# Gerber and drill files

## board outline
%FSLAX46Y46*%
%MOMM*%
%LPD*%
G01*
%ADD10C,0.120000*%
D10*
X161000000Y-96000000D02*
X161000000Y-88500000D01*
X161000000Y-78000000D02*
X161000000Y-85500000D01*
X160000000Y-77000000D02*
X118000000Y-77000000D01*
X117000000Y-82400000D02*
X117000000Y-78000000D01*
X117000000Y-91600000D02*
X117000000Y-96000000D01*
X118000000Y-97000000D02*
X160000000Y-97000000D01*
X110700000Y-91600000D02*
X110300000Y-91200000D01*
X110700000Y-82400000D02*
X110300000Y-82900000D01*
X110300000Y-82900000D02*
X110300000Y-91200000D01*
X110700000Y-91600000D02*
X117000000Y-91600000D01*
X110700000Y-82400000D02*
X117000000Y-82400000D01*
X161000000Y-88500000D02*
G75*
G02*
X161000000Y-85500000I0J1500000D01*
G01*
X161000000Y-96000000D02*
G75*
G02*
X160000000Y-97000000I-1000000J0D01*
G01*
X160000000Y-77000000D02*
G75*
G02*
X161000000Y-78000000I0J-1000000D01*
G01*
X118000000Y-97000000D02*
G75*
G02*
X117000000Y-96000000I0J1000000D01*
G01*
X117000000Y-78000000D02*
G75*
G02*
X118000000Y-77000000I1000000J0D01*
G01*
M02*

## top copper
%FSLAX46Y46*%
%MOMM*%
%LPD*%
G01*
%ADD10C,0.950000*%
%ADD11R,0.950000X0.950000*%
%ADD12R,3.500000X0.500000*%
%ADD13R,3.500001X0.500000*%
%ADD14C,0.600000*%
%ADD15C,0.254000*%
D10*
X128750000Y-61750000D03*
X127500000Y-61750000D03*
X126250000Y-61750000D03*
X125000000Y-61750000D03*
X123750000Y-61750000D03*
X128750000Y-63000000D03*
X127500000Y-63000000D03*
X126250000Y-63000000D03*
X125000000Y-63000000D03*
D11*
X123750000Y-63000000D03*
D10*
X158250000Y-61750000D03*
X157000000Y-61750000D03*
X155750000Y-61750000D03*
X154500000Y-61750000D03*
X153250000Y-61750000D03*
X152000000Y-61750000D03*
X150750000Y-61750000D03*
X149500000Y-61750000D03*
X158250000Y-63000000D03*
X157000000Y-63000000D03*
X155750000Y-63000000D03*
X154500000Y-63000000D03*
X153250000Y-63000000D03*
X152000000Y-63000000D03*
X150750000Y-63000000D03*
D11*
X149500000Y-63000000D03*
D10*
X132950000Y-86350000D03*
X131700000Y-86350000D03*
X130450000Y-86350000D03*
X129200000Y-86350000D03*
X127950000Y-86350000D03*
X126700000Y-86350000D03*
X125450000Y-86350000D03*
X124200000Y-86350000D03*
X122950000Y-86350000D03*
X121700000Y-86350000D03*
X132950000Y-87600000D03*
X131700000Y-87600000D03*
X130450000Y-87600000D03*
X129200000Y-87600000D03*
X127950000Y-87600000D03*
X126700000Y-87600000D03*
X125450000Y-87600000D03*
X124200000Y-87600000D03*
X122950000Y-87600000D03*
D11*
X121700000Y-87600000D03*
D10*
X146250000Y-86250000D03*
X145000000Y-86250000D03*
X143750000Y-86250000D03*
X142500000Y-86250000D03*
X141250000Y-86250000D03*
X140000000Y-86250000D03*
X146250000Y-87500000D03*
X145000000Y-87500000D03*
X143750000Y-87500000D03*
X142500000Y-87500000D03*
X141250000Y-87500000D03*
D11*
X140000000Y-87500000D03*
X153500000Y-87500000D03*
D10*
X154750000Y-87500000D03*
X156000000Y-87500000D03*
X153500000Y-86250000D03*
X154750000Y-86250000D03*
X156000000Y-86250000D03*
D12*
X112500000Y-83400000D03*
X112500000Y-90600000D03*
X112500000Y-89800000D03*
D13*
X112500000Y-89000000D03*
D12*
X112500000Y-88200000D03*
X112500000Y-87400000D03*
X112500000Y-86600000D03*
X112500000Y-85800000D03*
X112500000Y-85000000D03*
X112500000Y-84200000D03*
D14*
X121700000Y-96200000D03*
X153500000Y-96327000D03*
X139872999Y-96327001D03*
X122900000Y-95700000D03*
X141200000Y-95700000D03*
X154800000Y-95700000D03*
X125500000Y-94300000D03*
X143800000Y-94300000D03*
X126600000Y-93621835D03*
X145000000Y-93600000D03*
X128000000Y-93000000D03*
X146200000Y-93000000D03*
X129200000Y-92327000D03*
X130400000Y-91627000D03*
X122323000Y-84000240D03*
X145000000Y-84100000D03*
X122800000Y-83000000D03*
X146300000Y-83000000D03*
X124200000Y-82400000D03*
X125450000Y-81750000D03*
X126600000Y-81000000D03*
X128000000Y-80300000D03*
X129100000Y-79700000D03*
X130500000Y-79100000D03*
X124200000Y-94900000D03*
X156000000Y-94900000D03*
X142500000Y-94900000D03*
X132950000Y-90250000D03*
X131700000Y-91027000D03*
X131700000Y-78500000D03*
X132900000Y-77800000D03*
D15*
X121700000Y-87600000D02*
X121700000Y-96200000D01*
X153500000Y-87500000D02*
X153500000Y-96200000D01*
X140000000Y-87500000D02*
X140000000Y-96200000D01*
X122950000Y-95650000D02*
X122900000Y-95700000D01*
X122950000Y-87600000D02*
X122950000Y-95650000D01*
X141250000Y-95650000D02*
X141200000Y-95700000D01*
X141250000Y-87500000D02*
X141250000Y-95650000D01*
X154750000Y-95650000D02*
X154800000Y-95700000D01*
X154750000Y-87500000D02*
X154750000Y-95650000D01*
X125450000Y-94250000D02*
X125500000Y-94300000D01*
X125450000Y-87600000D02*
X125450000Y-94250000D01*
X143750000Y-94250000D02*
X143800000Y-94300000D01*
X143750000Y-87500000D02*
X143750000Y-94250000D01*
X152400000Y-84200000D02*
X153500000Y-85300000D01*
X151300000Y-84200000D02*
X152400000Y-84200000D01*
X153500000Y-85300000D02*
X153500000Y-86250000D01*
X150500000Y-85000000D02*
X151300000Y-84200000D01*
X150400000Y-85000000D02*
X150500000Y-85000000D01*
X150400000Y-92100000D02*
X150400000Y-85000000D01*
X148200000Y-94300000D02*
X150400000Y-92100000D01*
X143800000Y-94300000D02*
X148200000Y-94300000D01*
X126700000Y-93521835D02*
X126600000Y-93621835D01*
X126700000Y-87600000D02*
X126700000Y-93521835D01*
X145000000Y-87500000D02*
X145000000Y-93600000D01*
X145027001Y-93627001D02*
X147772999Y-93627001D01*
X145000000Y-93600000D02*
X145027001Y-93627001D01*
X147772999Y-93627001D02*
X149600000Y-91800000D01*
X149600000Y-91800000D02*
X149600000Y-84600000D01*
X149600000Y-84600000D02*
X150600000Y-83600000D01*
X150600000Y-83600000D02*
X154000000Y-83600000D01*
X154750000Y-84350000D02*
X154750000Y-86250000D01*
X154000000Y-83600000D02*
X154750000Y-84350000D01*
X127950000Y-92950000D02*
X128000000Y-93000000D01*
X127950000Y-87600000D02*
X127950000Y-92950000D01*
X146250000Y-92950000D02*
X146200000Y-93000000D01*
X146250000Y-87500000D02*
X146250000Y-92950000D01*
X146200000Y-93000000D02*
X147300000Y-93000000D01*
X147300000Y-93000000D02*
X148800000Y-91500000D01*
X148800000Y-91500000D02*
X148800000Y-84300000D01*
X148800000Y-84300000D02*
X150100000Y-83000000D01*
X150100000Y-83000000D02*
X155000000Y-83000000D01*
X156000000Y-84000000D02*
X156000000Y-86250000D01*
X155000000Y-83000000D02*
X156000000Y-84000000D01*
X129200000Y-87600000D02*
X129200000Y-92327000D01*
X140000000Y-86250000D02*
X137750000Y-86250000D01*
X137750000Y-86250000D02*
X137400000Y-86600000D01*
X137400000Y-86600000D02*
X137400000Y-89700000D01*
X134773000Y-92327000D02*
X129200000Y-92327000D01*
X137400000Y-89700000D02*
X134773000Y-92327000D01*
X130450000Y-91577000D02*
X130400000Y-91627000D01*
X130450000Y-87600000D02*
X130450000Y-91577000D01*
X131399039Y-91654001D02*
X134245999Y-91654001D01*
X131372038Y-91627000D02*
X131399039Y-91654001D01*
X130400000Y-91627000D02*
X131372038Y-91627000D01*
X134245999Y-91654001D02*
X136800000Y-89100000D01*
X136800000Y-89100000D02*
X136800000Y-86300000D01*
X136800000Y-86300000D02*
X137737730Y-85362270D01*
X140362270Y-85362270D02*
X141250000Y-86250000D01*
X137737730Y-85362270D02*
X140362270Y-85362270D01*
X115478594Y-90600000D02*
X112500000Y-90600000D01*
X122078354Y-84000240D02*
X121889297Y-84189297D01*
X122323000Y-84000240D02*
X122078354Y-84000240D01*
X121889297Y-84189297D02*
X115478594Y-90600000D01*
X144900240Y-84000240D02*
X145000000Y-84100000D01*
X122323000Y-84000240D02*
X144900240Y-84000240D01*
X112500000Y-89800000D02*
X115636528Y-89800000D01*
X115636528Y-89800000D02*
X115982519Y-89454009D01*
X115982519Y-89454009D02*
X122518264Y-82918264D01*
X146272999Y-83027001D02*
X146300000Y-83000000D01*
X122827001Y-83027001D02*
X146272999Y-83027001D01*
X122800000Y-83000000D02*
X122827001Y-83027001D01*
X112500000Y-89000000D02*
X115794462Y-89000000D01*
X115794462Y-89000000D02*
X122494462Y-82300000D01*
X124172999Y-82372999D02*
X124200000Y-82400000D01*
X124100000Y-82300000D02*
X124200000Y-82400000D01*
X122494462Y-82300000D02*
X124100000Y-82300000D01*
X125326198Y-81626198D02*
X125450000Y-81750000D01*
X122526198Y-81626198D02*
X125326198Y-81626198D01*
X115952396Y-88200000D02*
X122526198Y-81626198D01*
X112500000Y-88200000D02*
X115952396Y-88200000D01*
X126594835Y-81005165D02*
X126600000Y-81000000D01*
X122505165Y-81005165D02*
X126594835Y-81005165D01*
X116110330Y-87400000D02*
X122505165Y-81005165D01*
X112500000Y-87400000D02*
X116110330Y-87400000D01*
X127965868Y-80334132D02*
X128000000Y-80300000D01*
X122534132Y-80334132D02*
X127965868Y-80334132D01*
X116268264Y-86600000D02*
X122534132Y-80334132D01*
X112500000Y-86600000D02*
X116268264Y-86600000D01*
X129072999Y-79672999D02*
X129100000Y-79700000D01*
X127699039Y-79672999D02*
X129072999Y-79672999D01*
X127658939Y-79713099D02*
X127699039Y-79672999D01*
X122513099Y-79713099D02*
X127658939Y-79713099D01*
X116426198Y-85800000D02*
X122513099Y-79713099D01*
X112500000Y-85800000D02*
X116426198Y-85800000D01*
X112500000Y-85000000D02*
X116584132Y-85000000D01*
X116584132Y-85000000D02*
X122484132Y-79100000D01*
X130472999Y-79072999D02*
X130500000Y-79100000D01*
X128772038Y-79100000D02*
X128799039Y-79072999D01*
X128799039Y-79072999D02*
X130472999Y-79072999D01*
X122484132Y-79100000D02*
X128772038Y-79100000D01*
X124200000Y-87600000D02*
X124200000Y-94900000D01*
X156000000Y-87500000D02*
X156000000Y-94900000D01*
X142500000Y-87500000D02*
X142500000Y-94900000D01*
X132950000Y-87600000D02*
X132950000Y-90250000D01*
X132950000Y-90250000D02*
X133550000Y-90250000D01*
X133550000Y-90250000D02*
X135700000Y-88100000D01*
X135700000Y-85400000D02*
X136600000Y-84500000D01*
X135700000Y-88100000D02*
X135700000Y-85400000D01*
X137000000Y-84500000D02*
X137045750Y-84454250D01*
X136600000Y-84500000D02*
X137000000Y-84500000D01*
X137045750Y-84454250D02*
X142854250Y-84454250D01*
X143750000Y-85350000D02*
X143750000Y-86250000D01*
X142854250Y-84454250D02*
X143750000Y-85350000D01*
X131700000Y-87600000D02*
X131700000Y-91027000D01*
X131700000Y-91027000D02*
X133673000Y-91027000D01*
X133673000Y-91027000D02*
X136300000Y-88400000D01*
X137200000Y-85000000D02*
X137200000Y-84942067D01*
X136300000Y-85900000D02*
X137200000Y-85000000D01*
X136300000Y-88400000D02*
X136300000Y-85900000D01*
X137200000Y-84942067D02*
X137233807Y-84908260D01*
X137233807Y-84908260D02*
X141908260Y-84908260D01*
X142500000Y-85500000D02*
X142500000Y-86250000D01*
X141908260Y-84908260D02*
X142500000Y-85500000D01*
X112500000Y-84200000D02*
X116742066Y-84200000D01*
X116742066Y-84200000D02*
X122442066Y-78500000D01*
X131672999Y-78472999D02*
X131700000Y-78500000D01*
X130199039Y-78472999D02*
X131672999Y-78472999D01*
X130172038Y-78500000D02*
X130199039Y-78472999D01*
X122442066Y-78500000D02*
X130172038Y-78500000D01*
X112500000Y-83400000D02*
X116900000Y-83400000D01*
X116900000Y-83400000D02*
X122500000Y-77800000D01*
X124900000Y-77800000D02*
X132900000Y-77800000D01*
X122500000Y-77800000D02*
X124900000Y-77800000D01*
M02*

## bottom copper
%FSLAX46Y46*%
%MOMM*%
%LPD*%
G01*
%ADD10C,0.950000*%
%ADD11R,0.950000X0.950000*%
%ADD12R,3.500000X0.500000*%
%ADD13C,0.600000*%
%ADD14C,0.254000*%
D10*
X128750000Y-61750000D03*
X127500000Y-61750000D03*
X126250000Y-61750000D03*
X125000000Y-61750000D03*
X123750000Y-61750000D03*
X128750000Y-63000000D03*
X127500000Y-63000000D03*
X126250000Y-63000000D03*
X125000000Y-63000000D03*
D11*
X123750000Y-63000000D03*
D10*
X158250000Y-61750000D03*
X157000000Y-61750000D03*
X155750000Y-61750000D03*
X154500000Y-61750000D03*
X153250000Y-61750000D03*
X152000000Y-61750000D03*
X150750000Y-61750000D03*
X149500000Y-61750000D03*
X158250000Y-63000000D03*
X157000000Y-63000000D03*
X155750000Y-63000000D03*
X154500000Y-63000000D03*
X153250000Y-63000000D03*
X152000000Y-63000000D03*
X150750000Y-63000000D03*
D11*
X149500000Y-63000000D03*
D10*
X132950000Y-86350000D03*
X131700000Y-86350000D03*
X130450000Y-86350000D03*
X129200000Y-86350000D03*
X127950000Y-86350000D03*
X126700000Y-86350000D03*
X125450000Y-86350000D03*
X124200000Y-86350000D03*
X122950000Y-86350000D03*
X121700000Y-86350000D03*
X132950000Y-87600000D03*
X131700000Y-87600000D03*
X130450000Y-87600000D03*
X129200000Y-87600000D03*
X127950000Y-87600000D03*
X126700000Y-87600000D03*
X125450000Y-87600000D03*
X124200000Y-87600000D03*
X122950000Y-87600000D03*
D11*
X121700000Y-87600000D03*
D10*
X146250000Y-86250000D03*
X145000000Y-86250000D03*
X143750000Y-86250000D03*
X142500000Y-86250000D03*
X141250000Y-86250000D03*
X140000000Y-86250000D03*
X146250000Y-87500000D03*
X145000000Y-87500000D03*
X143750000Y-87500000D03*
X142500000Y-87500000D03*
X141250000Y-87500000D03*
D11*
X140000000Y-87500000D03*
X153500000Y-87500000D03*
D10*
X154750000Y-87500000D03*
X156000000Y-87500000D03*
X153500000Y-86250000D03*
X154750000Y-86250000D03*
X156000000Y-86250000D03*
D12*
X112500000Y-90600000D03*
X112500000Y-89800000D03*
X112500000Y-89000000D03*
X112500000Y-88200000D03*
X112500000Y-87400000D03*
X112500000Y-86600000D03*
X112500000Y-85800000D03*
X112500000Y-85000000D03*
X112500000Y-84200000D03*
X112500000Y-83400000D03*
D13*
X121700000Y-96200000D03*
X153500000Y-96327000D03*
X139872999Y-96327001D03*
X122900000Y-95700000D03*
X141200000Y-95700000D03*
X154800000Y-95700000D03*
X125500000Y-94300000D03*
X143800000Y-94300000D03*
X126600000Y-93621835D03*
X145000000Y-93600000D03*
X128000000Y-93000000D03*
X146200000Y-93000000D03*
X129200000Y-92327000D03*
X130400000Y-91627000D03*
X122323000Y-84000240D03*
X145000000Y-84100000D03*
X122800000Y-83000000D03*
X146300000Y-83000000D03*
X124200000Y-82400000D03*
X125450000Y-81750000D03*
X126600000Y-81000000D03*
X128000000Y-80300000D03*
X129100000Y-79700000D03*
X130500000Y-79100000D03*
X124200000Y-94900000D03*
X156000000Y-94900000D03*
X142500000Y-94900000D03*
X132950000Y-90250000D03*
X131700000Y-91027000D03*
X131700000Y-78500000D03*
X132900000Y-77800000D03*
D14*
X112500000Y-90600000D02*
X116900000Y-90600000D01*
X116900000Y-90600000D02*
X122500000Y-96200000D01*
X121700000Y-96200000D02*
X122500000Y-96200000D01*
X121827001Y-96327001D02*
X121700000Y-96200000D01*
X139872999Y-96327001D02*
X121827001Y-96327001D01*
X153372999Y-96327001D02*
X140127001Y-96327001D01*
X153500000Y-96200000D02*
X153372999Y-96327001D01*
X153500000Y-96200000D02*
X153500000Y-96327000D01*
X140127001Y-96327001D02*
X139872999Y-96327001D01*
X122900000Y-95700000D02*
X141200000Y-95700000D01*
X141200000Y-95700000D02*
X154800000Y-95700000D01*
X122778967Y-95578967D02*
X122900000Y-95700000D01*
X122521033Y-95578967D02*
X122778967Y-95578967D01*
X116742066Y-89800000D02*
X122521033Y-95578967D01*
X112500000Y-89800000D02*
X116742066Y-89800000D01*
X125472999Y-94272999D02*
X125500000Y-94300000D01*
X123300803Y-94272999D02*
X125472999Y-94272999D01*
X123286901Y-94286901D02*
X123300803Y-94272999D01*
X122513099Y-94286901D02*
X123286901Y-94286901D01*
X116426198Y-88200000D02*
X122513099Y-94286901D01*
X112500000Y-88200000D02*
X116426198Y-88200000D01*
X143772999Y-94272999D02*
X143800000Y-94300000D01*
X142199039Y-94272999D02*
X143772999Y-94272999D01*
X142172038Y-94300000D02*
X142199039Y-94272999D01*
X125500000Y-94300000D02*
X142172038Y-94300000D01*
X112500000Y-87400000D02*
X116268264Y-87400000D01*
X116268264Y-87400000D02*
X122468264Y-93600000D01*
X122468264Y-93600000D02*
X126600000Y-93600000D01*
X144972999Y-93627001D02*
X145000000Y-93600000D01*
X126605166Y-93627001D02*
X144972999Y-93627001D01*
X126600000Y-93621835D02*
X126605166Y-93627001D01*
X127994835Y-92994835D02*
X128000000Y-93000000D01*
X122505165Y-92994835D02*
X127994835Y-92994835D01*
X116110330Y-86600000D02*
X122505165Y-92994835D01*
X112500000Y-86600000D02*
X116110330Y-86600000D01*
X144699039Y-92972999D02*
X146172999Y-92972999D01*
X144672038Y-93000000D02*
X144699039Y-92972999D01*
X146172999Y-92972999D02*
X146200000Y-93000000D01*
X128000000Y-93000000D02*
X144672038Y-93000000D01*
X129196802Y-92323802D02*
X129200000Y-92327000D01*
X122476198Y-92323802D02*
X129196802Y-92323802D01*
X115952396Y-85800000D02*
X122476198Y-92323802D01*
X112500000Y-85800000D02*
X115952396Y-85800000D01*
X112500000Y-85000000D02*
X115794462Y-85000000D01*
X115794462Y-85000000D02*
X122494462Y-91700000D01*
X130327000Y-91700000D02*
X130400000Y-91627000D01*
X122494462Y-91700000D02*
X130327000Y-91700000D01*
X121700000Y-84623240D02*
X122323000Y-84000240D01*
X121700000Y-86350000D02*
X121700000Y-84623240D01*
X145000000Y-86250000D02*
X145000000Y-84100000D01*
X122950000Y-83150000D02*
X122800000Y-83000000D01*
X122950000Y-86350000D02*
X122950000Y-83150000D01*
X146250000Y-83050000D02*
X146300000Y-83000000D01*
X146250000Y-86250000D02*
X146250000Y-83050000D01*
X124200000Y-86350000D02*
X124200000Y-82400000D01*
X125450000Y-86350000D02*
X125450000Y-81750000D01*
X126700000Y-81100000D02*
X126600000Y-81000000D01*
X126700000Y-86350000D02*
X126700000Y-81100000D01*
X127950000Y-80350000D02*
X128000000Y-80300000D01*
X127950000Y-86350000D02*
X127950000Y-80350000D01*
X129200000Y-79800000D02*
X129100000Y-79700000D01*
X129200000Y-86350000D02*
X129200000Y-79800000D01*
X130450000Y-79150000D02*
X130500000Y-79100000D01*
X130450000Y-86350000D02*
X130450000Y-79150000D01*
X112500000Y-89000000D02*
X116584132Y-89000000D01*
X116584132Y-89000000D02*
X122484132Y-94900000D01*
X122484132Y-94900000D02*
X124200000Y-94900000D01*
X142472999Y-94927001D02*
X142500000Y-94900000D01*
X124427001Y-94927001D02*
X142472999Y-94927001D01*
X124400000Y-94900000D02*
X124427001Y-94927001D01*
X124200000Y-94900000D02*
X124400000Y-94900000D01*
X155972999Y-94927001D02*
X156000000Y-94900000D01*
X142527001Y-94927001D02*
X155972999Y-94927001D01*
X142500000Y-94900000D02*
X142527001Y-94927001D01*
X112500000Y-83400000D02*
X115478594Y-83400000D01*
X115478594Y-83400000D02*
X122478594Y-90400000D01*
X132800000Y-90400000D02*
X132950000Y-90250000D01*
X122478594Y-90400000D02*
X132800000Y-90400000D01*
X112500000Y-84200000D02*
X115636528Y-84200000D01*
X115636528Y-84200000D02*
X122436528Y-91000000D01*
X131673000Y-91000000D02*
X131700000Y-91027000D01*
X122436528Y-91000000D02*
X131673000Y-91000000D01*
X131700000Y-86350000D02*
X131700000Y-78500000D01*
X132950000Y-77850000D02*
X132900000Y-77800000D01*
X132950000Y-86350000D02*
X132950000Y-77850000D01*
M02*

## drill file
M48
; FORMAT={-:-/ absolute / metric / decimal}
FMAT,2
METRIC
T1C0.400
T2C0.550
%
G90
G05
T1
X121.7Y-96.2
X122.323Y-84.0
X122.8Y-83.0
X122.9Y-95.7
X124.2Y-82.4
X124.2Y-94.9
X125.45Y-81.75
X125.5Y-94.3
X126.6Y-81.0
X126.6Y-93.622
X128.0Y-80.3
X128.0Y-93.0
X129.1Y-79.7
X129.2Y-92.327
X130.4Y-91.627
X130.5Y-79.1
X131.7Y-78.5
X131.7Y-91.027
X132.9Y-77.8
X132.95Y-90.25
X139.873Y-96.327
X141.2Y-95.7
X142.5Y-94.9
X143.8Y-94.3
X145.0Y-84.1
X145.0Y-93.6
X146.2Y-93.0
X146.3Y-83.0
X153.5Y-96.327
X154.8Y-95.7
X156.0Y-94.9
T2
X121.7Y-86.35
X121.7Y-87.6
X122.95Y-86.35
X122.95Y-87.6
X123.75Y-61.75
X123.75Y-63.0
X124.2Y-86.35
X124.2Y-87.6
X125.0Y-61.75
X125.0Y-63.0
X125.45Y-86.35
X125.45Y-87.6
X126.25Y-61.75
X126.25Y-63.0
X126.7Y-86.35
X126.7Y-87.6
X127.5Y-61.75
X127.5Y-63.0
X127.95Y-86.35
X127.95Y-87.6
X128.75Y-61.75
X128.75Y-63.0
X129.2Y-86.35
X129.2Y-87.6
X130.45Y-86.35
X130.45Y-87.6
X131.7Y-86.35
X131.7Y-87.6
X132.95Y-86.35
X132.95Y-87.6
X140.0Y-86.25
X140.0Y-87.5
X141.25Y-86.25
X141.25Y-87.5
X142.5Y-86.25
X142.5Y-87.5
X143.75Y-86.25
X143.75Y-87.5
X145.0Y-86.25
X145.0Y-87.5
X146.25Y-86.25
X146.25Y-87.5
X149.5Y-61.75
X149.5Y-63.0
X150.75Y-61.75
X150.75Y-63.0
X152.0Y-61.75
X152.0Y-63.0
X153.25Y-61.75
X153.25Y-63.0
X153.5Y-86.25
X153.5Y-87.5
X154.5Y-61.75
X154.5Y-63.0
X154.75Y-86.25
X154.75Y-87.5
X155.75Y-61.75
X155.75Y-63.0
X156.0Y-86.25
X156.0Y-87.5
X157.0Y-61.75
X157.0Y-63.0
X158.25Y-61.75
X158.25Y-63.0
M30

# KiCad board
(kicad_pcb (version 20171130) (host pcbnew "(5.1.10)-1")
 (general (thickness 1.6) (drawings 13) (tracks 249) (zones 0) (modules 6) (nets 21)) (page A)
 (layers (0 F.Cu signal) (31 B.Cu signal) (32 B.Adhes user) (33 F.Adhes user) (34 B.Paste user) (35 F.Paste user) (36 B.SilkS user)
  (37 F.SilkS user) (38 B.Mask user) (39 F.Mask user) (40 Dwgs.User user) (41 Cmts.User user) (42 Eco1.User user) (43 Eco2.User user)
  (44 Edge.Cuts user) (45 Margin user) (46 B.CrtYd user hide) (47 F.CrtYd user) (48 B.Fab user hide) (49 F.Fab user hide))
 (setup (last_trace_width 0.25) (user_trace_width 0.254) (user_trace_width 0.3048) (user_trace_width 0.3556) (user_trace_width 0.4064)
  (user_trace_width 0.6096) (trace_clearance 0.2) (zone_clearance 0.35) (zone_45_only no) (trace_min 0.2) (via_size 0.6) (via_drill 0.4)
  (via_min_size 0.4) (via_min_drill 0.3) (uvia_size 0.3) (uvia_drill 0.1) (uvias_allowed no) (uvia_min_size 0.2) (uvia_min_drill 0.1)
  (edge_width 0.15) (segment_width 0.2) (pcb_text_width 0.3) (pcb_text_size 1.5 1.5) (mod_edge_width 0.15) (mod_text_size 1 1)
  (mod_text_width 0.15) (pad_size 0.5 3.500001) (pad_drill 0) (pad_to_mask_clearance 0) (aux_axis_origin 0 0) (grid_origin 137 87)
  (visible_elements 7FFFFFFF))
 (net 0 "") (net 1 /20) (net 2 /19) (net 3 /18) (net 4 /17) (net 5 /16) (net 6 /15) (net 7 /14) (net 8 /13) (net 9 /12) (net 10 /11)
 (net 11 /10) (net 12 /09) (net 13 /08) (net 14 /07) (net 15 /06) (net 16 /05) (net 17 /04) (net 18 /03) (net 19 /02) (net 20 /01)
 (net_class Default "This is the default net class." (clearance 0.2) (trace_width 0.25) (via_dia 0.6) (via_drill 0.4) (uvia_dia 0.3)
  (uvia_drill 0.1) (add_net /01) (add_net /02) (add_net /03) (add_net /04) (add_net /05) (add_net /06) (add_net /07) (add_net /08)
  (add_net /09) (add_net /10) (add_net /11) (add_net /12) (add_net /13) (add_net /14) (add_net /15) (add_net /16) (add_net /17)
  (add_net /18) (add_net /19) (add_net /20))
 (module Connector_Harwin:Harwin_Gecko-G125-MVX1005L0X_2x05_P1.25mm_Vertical (layer F.Cu) (at 123.75 63)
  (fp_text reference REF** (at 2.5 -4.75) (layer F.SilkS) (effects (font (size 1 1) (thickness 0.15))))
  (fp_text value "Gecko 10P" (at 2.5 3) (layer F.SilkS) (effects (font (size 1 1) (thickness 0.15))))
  (pad 10 thru_hole circle (at 5 -1.25) (size 0.95 0.95) (drill 0.55) (layers *.Cu *.Mask))
  (pad 9 thru_hole circle (at 3.75 -1.25) (size 0.95 0.95) (drill 0.55) (layers *.Cu *.Mask))
  (pad 8 thru_hole circle (at 2.5 -1.25) (size 0.95 0.95) (drill 0.55) (layers *.Cu *.Mask))
  (pad 7 thru_hole circle (at 1.25 -1.25) (size 0.95 0.95) (drill 0.55) (layers *.Cu *.Mask))
  (pad 6 thru_hole circle (at 0 -1.25) (size 0.95 0.95) (drill 0.55) (layers *.Cu *.Mask))
  (pad 5 thru_hole circle (at 5 0) (size 0.95 0.95) (drill 0.55) (layers *.Cu *.Mask))
  (pad 4 thru_hole circle (at 3.75 0) (size 0.95 0.95) (drill 0.55) (layers *.Cu *.Mask))
  (pad 3 thru_hole circle (at 2.5 0) (size 0.95 0.95) (drill 0.55) (layers *.Cu *.Mask))
  (pad 2 thru_hole circle (at 1.25 0) (size 0.95 0.95) (drill 0.55) (layers *.Cu *.Mask))
  (pad 1 thru_hole rect (at 0 0) (size 0.95 0.95) (drill 0.55) (layers *.Cu *.Mask)))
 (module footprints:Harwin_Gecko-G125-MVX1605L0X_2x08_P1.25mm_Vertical (layer F.Cu) (at 149.5 63)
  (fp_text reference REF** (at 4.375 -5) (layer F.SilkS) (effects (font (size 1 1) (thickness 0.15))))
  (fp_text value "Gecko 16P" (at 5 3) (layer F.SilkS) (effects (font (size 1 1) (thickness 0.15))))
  (pad 16 thru_hole circle (at 8.75 -1.25) (size 0.95 0.95) (drill 0.55) (layers *.Cu *.Mask))
  (pad 15 thru_hole circle (at 7.5 -1.25) (size 0.95 0.95) (drill 0.55) (layers *.Cu *.Mask))
  (pad 14 thru_hole circle (at 6.25 -1.25) (size 0.95 0.95) (drill 0.55) (layers *.Cu *.Mask))
  (pad 13 thru_hole circle (at 5 -1.25) (size 0.95 0.95) (drill 0.55) (layers *.Cu *.Mask))
  (pad 12 thru_hole circle (at 3.75 -1.25) (size 0.95 0.95) (drill 0.55) (layers *.Cu *.Mask))
  (pad 11 thru_hole circle (at 2.5 -1.25) (size 0.95 0.95) (drill 0.55) (layers *.Cu *.Mask))
  (pad 10 thru_hole circle (at 1.25 -1.25) (size 0.95 0.95) (drill 0.55) (layers *.Cu *.Mask))
  (pad 9 thru_hole circle (at 0 -1.25) (size 0.95 0.95) (drill 0.55) (layers *.Cu *.Mask))
  (pad 8 thru_hole circle (at 8.75 0) (size 0.95 0.95) (drill 0.55) (layers *.Cu *.Mask))
  (pad 7 thru_hole circle (at 7.5 0) (size 0.95 0.95) (drill 0.55) (layers *.Cu *.Mask))
  (pad 6 thru_hole circle (at 6.25 0) (size 0.95 0.95) (drill 0.55) (layers *.Cu *.Mask))
  (pad 5 thru_hole circle (at 5 0) (size 0.95 0.95) (drill 0.55) (layers *.Cu *.Mask))
  (pad 4 thru_hole circle (at 3.75 0) (size 0.95 0.95) (drill 0.55) (layers *.Cu *.Mask))
  (pad 3 thru_hole circle (at 2.5 0) (size 0.95 0.95) (drill 0.55) (layers *.Cu *.Mask))
  (pad 2 thru_hole circle (at 1.25 0) (size 0.95 0.95) (drill 0.55) (layers *.Cu *.Mask))
  (pad 1 thru_hole rect (at 0 0) (size 0.95 0.95) (drill 0.55) (layers *.Cu *.Mask)))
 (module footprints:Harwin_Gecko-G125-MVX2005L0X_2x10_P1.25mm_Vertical (layer F.Cu) (at 121.7 87.6)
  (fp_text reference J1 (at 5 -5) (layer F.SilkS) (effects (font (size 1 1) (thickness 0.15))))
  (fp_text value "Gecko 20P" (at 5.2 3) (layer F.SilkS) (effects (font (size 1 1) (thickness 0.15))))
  (pad 20 thru_hole circle (at 11.25 -1.25) (size 0.95 0.95) (drill 0.55) (layers *.Cu *.Mask) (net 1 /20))
  (pad 19 thru_hole circle (at 10 -1.25) (size 0.95 0.95) (drill 0.55) (layers *.Cu *.Mask) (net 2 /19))
  (pad 18 thru_hole circle (at 8.75 -1.25) (size 0.95 0.95) (drill 0.55) (layers *.Cu *.Mask) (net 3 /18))
  (pad 17 thru_hole circle (at 7.5 -1.25) (size 0.95 0.95) (drill 0.55) (layers *.Cu *.Mask) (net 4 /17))
  (pad 16 thru_hole circle (at 6.25 -1.25) (size 0.95 0.95) (drill 0.55) (layers *.Cu *.Mask) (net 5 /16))
  (pad 15 thru_hole circle (at 5 -1.25) (size 0.95 0.95) (drill 0.55) (layers *.Cu *.Mask) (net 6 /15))
  (pad 14 thru_hole circle (at 3.75 -1.25) (size 0.95 0.95) (drill 0.55) (layers *.Cu *.Mask) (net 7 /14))
  (pad 13 thru_hole circle (at 2.5 -1.25) (size 0.95 0.95) (drill 0.55) (layers *.Cu *.Mask) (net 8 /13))
  (pad 12 thru_hole circle (at 1.25 -1.25) (size 0.95 0.95) (drill 0.55) (layers *.Cu *.Mask) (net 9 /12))
  (pad 11 thru_hole circle (at 0 -1.25) (size 0.95 0.95) (drill 0.55) (layers *.Cu *.Mask) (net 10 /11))
  (pad 10 thru_hole circle (at 11.25 0) (size 0.95 0.95) (drill 0.55) (layers *.Cu *.Mask) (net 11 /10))
  (pad 9 thru_hole circle (at 10 0) (size 0.95 0.95) (drill 0.55) (layers *.Cu *.Mask) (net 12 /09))
  (pad 8 thru_hole circle (at 8.75 0) (size 0.95 0.95) (drill 0.55) (layers *.Cu *.Mask) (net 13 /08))
  (pad 7 thru_hole circle (at 7.5 0) (size 0.95 0.95) (drill 0.55) (layers *.Cu *.Mask) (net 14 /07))
  (pad 6 thru_hole circle (at 6.25 0) (size 0.95 0.95) (drill 0.55) (layers *.Cu *.Mask) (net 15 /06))
  (pad 5 thru_hole circle (at 5 0) (size 0.95 0.95) (drill 0.55) (layers *.Cu *.Mask) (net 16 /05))
  (pad 4 thru_hole circle (at 3.75 0) (size 0.95 0.95) (drill 0.55) (layers *.Cu *.Mask) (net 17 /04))
  (pad 3 thru_hole circle (at 2.5 0) (size 0.95 0.95) (drill 0.55) (layers *.Cu *.Mask) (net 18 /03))
  (pad 2 thru_hole circle (at 1.25 0) (size 0.95 0.95) (drill 0.55) (layers *.Cu *.Mask) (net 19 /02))
  (pad 1 thru_hole rect (at 0 0) (size 0.95 0.95) (drill 0.55) (layers *.Cu *.Mask) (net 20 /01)))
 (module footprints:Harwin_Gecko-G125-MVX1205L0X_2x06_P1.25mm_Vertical (layer F.Cu) (at 140 87.5)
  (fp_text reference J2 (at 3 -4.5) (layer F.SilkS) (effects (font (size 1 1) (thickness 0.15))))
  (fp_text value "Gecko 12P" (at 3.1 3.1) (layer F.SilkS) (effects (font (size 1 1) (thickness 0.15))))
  (pad 12 thru_hole circle (at 6.25 -1.25) (size 0.95 0.95) (drill 0.55) (layers *.Cu *.Mask) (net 9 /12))
  (pad 11 thru_hole circle (at 5 -1.25) (size 0.95 0.95) (drill 0.55) (layers *.Cu *.Mask) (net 10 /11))
  (pad 10 thru_hole circle (at 3.75 -1.25) (size 0.95 0.95) (drill 0.55) (layers *.Cu *.Mask) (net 11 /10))
  (pad 9 thru_hole circle (at 2.5 -1.25) (size 0.95 0.95) (drill 0.55) (layers *.Cu *.Mask) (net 12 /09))
  (pad 8 thru_hole circle (at 1.25 -1.25) (size 0.95 0.95) (drill 0.55) (layers *.Cu *.Mask) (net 13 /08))
  (pad 7 thru_hole circle (at 0 -1.25) (size 0.95 0.95) (drill 0.55) (layers *.Cu *.Mask) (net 14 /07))
  (pad 6 thru_hole circle (at 6.25 0) (size 0.95 0.95) (drill 0.55) (layers *.Cu *.Mask) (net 15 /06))
  (pad 5 thru_hole circle (at 5 0) (size 0.95 0.95) (drill 0.55) (layers *.Cu *.Mask) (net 16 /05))
  (pad 4 thru_hole circle (at 3.75 0) (size 0.95 0.95) (drill 0.55) (layers *.Cu *.Mask) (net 17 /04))
  (pad 3 thru_hole circle (at 2.5 0) (size 0.95 0.95) (drill 0.55) (layers *.Cu *.Mask) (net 18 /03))
  (pad 2 thru_hole circle (at 1.25 0) (size 0.95 0.95) (drill 0.55) (layers *.Cu *.Mask) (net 19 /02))
  (pad 1 thru_hole rect (at 0 0) (size 0.95 0.95) (drill 0.55) (layers *.Cu *.Mask) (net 20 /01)))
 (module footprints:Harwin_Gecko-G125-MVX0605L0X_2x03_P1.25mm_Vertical (layer F.Cu) (at 153.5 87.5)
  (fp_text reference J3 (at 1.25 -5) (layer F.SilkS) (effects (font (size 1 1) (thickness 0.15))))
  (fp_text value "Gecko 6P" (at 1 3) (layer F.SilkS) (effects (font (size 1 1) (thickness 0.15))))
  (pad 1 thru_hole rect (at 0 0) (size 0.95 0.95) (drill 0.55) (layers *.Cu *.Mask) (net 20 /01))
  (pad 2 thru_hole circle (at 1.25 0) (size 0.95 0.95) (drill 0.55) (layers *.Cu *.Mask) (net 19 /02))
  (pad 3 thru_hole circle (at 2.5 0) (size 0.95 0.95) (drill 0.55) (layers *.Cu *.Mask) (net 18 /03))
  (pad 4 thru_hole circle (at 0 -1.25) (size 0.95 0.95) (drill 0.55) (layers *.Cu *.Mask) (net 17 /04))
  (pad 5 thru_hole circle (at 1.25 -1.25) (size 0.95 0.95) (drill 0.55) (layers *.Cu *.Mask) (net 16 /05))
  (pad 6 thru_hole circle (at 2.5 -1.25) (size 0.95 0.95) (drill 0.55) (layers *.Cu *.Mask) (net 15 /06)))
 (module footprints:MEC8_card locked (layer F.Cu) (at 112.5 87 90)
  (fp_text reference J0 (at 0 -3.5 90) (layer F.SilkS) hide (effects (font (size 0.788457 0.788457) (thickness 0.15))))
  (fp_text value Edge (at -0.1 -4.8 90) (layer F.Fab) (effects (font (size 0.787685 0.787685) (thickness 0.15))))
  (fp_line (start -9 48.5) (end -1.5 48.5) (layer Edge.Cuts) (width 0.12))
  (fp_line (start 9 48.5) (end 1.5 48.5) (layer Edge.Cuts) (width 0.12))
  (fp_line (start 10 47.5) (end 10 5.5) (layer Edge.Cuts) (width 0.12))
  (fp_line (start 4.6 4.5) (end 9 4.5) (layer Edge.Cuts) (width 0.12))
  (fp_line (start -4.6 4.5) (end -9 4.5) (layer Edge.Cuts) (width 0.12))
  (fp_line (start -10 5.5) (end -10 47.5) (layer Edge.Cuts) (width 0.12))
  (fp_line (start -4.6 -1.8) (end -4.2 -2.2) (layer Edge.Cuts) (width 0.12))
  (fp_line (start 4.6 -1.8) (end 4.1 -2.2) (layer Edge.Cuts) (width 0.12))
  (fp_line (start 4.1 -2.2) (end -4.2 -2.2) (layer Edge.Cuts) (width 0.12))
  (fp_line (start -4.6 -1.8) (end -4.6 4.5) (layer Edge.Cuts) (width 0.12))
  (fp_line (start 4.6 -1.8) (end 4.6 4.5) (layer Edge.Cuts) (width 0.12))
  (fp_arc (start 0 48.5) (end 1.5 48.5) (angle -180) (layer Edge.Cuts) (width 0.12))
  (fp_arc (start -9 47.5) (end -10 47.5) (angle -90) (layer Edge.Cuts) (width 0.12))
  (fp_arc (start 9 47.5) (end 9 48.5) (angle -90) (layer Edge.Cuts) (width 0.12))
  (fp_arc (start -9 5.5) (end -9 4.5) (angle -90) (layer Edge.Cuts) (width 0.12))
  (fp_arc (start 9 5.5) (end 10 5.5) (angle -90) (layer Edge.Cuts) (width 0.12))
  (pad 20 smd rect (at 3.6 0 90) (size 0.5 3.5) (layers F.Cu F.Paste F.Mask) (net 1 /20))
  (pad 11 smd rect (at -3.6 0 90) (size 0.5 3.5) (layers F.Cu F.Paste F.Mask) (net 10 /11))
  (pad 12 smd rect (at -2.8 0 90) (size 0.5 3.5) (layers F.Cu F.Paste F.Mask) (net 9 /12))
  (pad 13 smd rect (at -2 0 90) (size 0.5 3.500001) (layers F.Cu F.Paste F.Mask) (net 8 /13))
  (pad 14 smd rect (at -1.2 0 90) (size 0.5 3.5) (layers F.Cu F.Paste F.Mask) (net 7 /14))
  (pad 15 smd rect (at -0.4 0 90) (size 0.5 3.5) (layers F.Cu F.Paste F.Mask) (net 6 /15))
  (pad 16 smd rect (at 0.4 0 90) (size 0.5 3.5) (layers F.Cu F.Paste F.Mask) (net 5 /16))
  (pad 17 smd rect (at 1.2 0 90) (size 0.5 3.5) (layers F.Cu F.Paste F.Mask) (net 4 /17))
  (pad 18 smd rect (at 2 0 90) (size 0.5 3.5) (layers F.Cu F.Paste F.Mask) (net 3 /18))
  (pad 19 smd rect (at 2.8 0 90) (size 0.5 3.5) (layers F.Cu F.Paste F.Mask) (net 2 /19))
  (pad 1 smd rect (at -3.6 0 90) (size 0.5 3.5) (layers B.Cu B.Paste B.Mask) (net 20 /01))
  (pad 2 smd rect (at -2.8 0 90) (size 0.5 3.5) (layers B.Cu B.Paste B.Mask) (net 19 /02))
  (pad 3 smd rect (at -2 0 90) (size 0.5 3.5) (layers B.Cu B.Paste B.Mask) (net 18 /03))
  (pad 4 smd rect (at -1.2 0 90) (size 0.5 3.5) (layers B.Cu B.Paste B.Mask) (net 17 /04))
  (pad 5 smd rect (at -0.4 0 90) (size 0.5 3.5) (layers B.Cu B.Paste B.Mask) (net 16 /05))
  (pad 6 smd rect (at 0.4 0 90) (size 0.5 3.5) (layers B.Cu B.Paste B.Mask) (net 15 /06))
  (pad 7 smd rect (at 1.2 0 90) (size 0.5 3.5) (layers B.Cu B.Paste B.Mask) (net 14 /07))
  (pad 8 smd rect (at 2 0 90) (size 0.5 3.5) (layers B.Cu B.Paste B.Mask) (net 13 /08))
  (pad 9 smd rect (at 2.8 0 90) (size 0.5 3.5) (layers B.Cu B.Paste B.Mask) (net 12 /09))
  (pad 10 smd rect (at 3.6 0 90) (size 0.5 3.5) (layers B.Cu B.Paste B.Mask) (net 11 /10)))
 (segment (start 112.5 90.6) (end 116.9 90.6) (width 0.254) (layer B.Cu) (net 20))
 (segment (start 116.9 90.6) (end 122.5 96.2) (width 0.254) (layer B.Cu) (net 20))
 (via (at 121.7 96.2) (size 0.6) (drill 0.4) (layers F.Cu B.Cu) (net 20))
 (segment (start 121.7 87.6) (end 121.7 96.2) (width 0.254) (layer F.Cu) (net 20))
 (segment (start 121.7 96.2) (end 122.5 96.2) (width 0.254) (layer B.Cu) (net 20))
 (segment (start 153.5 87.5) (end 153.5 96.2) (width 0.254) (layer F.Cu) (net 20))
 (segment (start 121.827001 96.327001) (end 121.7 96.2) (width 0.254) (layer B.Cu) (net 20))
 (segment (start 139.872999 96.327001) (end 121.827001 96.327001) (width 0.254) (layer B.Cu) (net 20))
 (segment (start 153.372999 96.327001) (end 140.127001 96.327001) (width 0.254) (layer B.Cu) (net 20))
 (segment (start 153.5 96.2) (end 153.372999 96.327001) (width 0.254) (layer B.Cu) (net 20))
 (segment (start 140 87.5) (end 140 96.2) (width 0.254) (layer F.Cu) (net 20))
 (via (at 153.5 96.327) (size 0.6) (drill 0.4) (layers F.Cu B.Cu) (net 20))
 (segment (start 153.5 96.2) (end 153.5 96.327) (width 0.254) (layer B.Cu) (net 20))
 (via (at 139.872999 96.327001) (size 0.6) (drill 0.4) (layers F.Cu B.Cu) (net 20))
 (segment (start 140.127001 96.327001) (end 139.872999 96.327001) (width 0.254) (layer B.Cu) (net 20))
 (segment (start 122.95 95.65) (end 122.9 95.7) (width 0.254) (layer F.Cu) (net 19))
 (via (at 122.9 95.7) (size 0.6) (drill 0.4) (layers F.Cu B.Cu) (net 19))
 (segment (start 122.95 87.6) (end 122.95 95.65) (width 0.254) (layer F.Cu) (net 19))
 (via (at 141.2 95.7) (size 0.6) (drill 0.4) (layers F.Cu B.Cu) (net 19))
 (segment (start 141.25 95.65) (end 141.2 95.7) (width 0.254) (layer F.Cu) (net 19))
 (segment (start 141.25 87.5) (end 141.25 95.65) (width 0.254) (layer F.Cu) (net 19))
 (via (at 154.8 95.7) (size 0.6) (drill 0.4) (layers F.Cu B.Cu) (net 19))
 (segment (start 154.75 95.65) (end 154.8 95.7) (width 0.254) (layer F.Cu) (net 19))
 (segment (start 154.75 87.5) (end 154.75 95.65) (width 0.254) (layer F.Cu) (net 19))
 (segment (start 122.9 95.7) (end 141.2 95.7) (width 0.254) (layer B.Cu) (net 19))
 (segment (start 141.2 95.7) (end 154.8 95.7) (width 0.254) (layer B.Cu) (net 19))
 (segment (start 122.778967 95.578967) (end 122.9 95.7) (width 0.254) (layer B.Cu) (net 19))
 (segment (start 122.521033 95.578967) (end 122.778967 95.578967) (width 0.254) (layer B.Cu) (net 19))
 (segment (start 116.742066 89.8) (end 122.521033 95.578967) (width 0.254) (layer B.Cu) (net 19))
 (segment (start 112.5 89.8) (end 116.742066 89.8) (width 0.254) (layer B.Cu) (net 19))
 (via (at 125.5 94.3) (size 0.6) (drill 0.4) (layers F.Cu B.Cu) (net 17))
 (segment (start 125.45 94.25) (end 125.5 94.3) (width 0.254) (layer F.Cu) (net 17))
 (segment (start 125.45 87.6) (end 125.45 94.25) (width 0.254) (layer F.Cu) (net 17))
 (segment (start 125.472999 94.272999) (end 125.5 94.3) (width 0.254) (layer B.Cu) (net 17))
 (segment (start 123.300803 94.272999) (end 125.472999 94.272999) (width 0.254) (layer B.Cu) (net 17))
 (segment (start 123.286901 94.286901) (end 123.300803 94.272999) (width 0.254) (layer B.Cu) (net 17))
 (segment (start 122.513099 94.286901) (end 123.286901 94.286901) (width 0.254) (layer B.Cu) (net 17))
 (segment (start 116.426198 88.2) (end 122.513099 94.286901) (width 0.254) (layer B.Cu) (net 17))
 (segment (start 112.5 88.2) (end 116.426198 88.2) (width 0.254) (layer B.Cu) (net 17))
 (via (at 143.8 94.3) (size 0.6) (drill 0.4) (layers F.Cu B.Cu) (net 17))
 (segment (start 143.75 94.25) (end 143.8 94.3) (width 0.254) (layer F.Cu) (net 17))
 (segment (start 143.75 87.5) (end 143.75 94.25) (width 0.254) (layer F.Cu) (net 17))
 (segment (start 143.772999 94.272999) (end 143.8 94.3) (width 0.254) (layer B.Cu) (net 17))
 (segment (start 142.199039 94.272999) (end 143.772999 94.272999) (width 0.254) (layer B.Cu) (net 17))
 (segment (start 142.172038 94.3) (end 142.199039 94.272999) (width 0.254) (layer B.Cu) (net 17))
 (segment (start 125.5 94.3) (end 142.172038 94.3) (width 0.254) (layer B.Cu) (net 17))
 (segment (start 152.4 84.2) (end 153.5 85.3) (width 0.254) (layer F.Cu) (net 17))
 (segment (start 151.3 84.2) (end 152.4 84.2) (width 0.254) (layer F.Cu) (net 17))
 (segment (start 153.5 85.3) (end 153.5 86.25) (width 0.254) (layer F.Cu) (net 17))
 (segment (start 150.5 85) (end 151.3 84.2) (width 0.254) (layer F.Cu) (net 17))
 (segment (start 150.4 85) (end 150.5 85) (width 0.254) (layer F.Cu) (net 17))
 (segment (start 150.4 92.1) (end 150.4 85) (width 0.254) (layer F.Cu) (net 17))
 (segment (start 148.2 94.3) (end 150.4 92.1) (width 0.254) (layer F.Cu) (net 17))
 (segment (start 143.8 94.3) (end 148.2 94.3) (width 0.254) (layer F.Cu) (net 17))
 (segment (start 112.5 87.4) (end 116.268264 87.4) (width 0.254) (layer B.Cu) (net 16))
 (segment (start 116.268264 87.4) (end 122.468264 93.6) (width 0.254) (layer B.Cu) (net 16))
 (segment (start 122.468264 93.6) (end 126.6 93.6) (width 0.254) (layer B.Cu) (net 16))
 (via (at 126.6 93.621835) (size 0.6) (drill 0.4) (layers F.Cu B.Cu) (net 16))
 (segment (start 126.7 93.521835) (end 126.6 93.621835) (width 0.254) (layer F.Cu) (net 16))
 (segment (start 126.7 87.6) (end 126.7 93.521835) (width 0.254) (layer F.Cu) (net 16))
 (via (at 145 93.6) (size 0.6) (drill 0.4) (layers F.Cu B.Cu) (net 16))
 (segment (start 145 87.5) (end 145 93.6) (width 0.254) (layer F.Cu) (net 16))
 (segment (start 144.972999 93.627001) (end 145 93.6) (width 0.254) (layer B.Cu) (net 16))
 (segment (start 126.605166 93.627001) (end 144.972999 93.627001) (width 0.254) (layer B.Cu) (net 16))
 (segment (start 126.6 93.621835) (end 126.605166 93.627001) (width 0.254) (layer B.Cu) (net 16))
 (segment (start 145.027001 93.627001) (end 147.772999 93.627001) (width 0.254) (layer F.Cu) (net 16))
 (segment (start 145 93.6) (end 145.027001 93.627001) (width 0.254) (layer F.Cu) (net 16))
 (segment (start 147.772999 93.627001) (end 149.6 91.8) (width 0.254) (layer F.Cu) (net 16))
 (segment (start 149.6 91.8) (end 149.6 84.6) (width 0.254) (layer F.Cu) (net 16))
 (segment (start 149.6 84.6) (end 150.6 83.6) (width 0.254) (layer F.Cu) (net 16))
 (segment (start 150.6 83.6) (end 154 83.6) (width 0.254) (layer F.Cu) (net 16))
 (segment (start 154.75 84.35) (end 154.75 86.25) (width 0.254) (layer F.Cu) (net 16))
 (segment (start 154 83.6) (end 154.75 84.35) (width 0.254) (layer F.Cu) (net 16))
 (via (at 128 93) (size 0.6) (drill 0.4) (layers F.Cu B.Cu) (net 15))
 (segment (start 127.95 92.95) (end 128 93) (width 0.254) (layer F.Cu) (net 15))
 (segment (start 127.95 87.6) (end 127.95 92.95) (width 0.254) (layer F.Cu) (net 15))
 (segment (start 127.994835 92.994835) (end 128 93) (width 0.254) (layer B.Cu) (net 15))
 (segment (start 122.505165 92.994835) (end 127.994835 92.994835) (width 0.254) (layer B.Cu) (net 15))
 (segment (start 116.11033 86.6) (end 122.505165 92.994835) (width 0.254) (layer B.Cu) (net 15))
 (segment (start 112.5 86.6) (end 116.11033 86.6) (width 0.254) (layer B.Cu) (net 15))
 (via (at 146.2 93) (size 0.6) (drill 0.4) (layers F.Cu B.Cu) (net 15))
 (segment (start 146.25 92.95) (end 146.2 93) (width 0.254) (layer F.Cu) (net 15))
 (segment (start 146.25 87.5) (end 146.25 92.95) (width 0.254) (layer F.Cu) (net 15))
 (segment (start 144.699039 92.972999) (end 146.172999 92.972999) (width 0.254) (layer B.Cu) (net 15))
 (segment (start 144.672038 93) (end 144.699039 92.972999) (width 0.254) (layer B.Cu) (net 15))
 (segment (start 146.172999 92.972999) (end 146.2 93) (width 0.254) (layer B.Cu) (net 15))
 (segment (start 128 93) (end 144.672038 93) (width 0.254) (layer B.Cu) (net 15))
 (segment (start 146.2 93) (end 147.3 93) (width 0.254) (layer F.Cu) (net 15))
 (segment (start 147.3 93) (end 148.8 91.5) (width 0.254) (layer F.Cu) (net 15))
 (segment (start 148.8 91.5) (end 148.8 84.3) (width 0.254) (layer F.Cu) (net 15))
 (segment (start 148.8 84.3) (end 150.1 83) (width 0.254) (layer F.Cu) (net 15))
 (segment (start 150.1 83) (end 155 83) (width 0.254) (layer F.Cu) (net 15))
 (segment (start 156 84) (end 156 86.25) (width 0.254) (layer F.Cu) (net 15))
 (segment (start 155 83) (end 156 84) (width 0.254) (layer F.Cu) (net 15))
 (via (at 129.2 92.327) (size 0.6) (drill 0.4) (layers F.Cu B.Cu) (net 14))
 (segment (start 129.2 87.6) (end 129.2 92.327) (width 0.254) (layer F.Cu) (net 14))
 (segment (start 129.196802 92.323802) (end 129.2 92.327) (width 0.254) (layer B.Cu) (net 14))
 (segment (start 122.476198 92.323802) (end 129.196802 92.323802) (width 0.254) (layer B.Cu) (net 14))
 (segment (start 115.952396 85.8) (end 122.476198 92.323802) (width 0.254) (layer B.Cu) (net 14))
 (segment (start 112.5 85.8) (end 115.952396 85.8) (width 0.254) (layer B.Cu) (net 14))
 (segment (start 140 86.25) (end 137.75 86.25) (width 0.254) (layer F.Cu) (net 14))
 (segment (start 137.75 86.25) (end 137.4 86.6) (width 0.254) (layer F.Cu) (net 14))
 (segment (start 137.4 86.6) (end 137.4 89.7) (width 0.254) (layer F.Cu) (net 14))
 (segment (start 134.773 92.327) (end 129.2 92.327) (width 0.254) (layer F.Cu) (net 14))
 (segment (start 137.4 89.7) (end 134.773 92.327) (width 0.254) (layer F.Cu) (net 14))
 (segment (start 112.5 85) (end 115.794462 85) (width 0.254) (layer B.Cu) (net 13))
 (segment (start 115.794462 85) (end 122.494462 91.7) (width 0.254) (layer B.Cu) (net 13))
 (via (at 130.4 91.627) (size 0.6) (drill 0.4) (layers F.Cu B.Cu) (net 13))
 (segment (start 130.45 91.577) (end 130.4 91.627) (width 0.254) (layer F.Cu) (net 13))
 (segment (start 130.45 87.6) (end 130.45 91.577) (width 0.254) (layer F.Cu) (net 13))
 (segment (start 130.327 91.7) (end 130.4 91.627) (width 0.254) (layer B.Cu) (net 13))
 (segment (start 122.494462 91.7) (end 130.327 91.7) (width 0.254) (layer B.Cu) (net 13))
 (segment (start 131.399039 91.654001) (end 134.245999 91.654001) (width 0.254) (layer F.Cu) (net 13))
 (segment (start 131.372038 91.627) (end 131.399039 91.654001) (width 0.254) (layer F.Cu) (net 13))
 (segment (start 130.4 91.627) (end 131.372038 91.627) (width 0.254) (layer F.Cu) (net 13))
 (segment (start 134.245999 91.654001) (end 136.8 89.1) (width 0.254) (layer F.Cu) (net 13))
 (segment (start 136.8 89.1) (end 136.8 86.3) (width 0.254) (layer F.Cu) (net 13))
 (segment (start 136.8 86.3) (end 137.73773 85.36227) (width 0.254) (layer F.Cu) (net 13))
 (segment (start 140.36227 85.36227) (end 141.25 86.25) (width 0.254) (layer F.Cu) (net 13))
 (segment (start 137.73773 85.36227) (end 140.36227 85.36227) (width 0.254) (layer F.Cu) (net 13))
 (segment (start 115.478594 90.6) (end 112.5 90.6) (width 0.254) (layer F.Cu) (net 10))
 (via (at 122.323 84.00024) (size 0.6) (drill 0.4) (layers F.Cu B.Cu) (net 10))
 (segment (start 121.7 84.62324) (end 122.323 84.00024) (width 0.254) (layer B.Cu) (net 10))
 (segment (start 121.7 86.35) (end 121.7 84.62324) (width 0.254) (layer B.Cu) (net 10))
 (segment (start 122.078354 84.00024) (end 121.889297 84.189297) (width 0.254) (layer F.Cu) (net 10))
 (segment (start 122.323 84.00024) (end 122.078354 84.00024) (width 0.254) (layer F.Cu) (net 10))
 (segment (start 121.889297 84.189297) (end 115.478594 90.6) (width 0.254) (layer F.Cu) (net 10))
 (via (at 145 84.1) (size 0.6) (drill 0.4) (layers F.Cu B.Cu) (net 10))
 (segment (start 145 86.25) (end 145 84.1) (width 0.254) (layer B.Cu) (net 10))
 (segment (start 144.90024 84.00024) (end 145 84.1) (width 0.254) (layer F.Cu) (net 10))
 (segment (start 122.323 84.00024) (end 144.90024 84.00024) (width 0.254) (layer F.Cu) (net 10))
 (segment (start 112.5 89.8) (end 115.636528 89.8) (width 0.254) (layer F.Cu) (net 9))
 (segment (start 115.636528 89.8) (end 115.982519 89.454009) (width 0.254) (layer F.Cu) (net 9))
 (segment (start 115.982519 89.454009) (end 122.518264 82.918264) (width 0.254) (layer F.Cu) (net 9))
 (via (at 122.8 83) (size 0.6) (drill 0.4) (layers F.Cu B.Cu) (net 9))
 (segment (start 122.95 83.15) (end 122.8 83) (width 0.254) (layer B.Cu) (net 9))
 (segment (start 122.95 86.35) (end 122.95 83.15) (width 0.254) (layer B.Cu) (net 9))
 (via (at 146.3 83) (size 0.6) (drill 0.4) (layers F.Cu B.Cu) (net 9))
 (segment (start 146.25 83.05) (end 146.3 83) (width 0.254) (layer B.Cu) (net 9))
 (segment (start 146.25 86.25) (end 146.25 83.05) (width 0.254) (layer B.Cu) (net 9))
 (segment (start 146.272999 83.027001) (end 146.3 83) (width 0.254) (layer F.Cu) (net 9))
 (segment (start 122.827001 83.027001) (end 146.272999 83.027001) (width 0.254) (layer F.Cu) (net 9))
 (segment (start 122.8 83) (end 122.827001 83.027001) (width 0.254) (layer F.Cu) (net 9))
 (segment (start 112.5 89) (end 115.794462 89) (width 0.254) (layer F.Cu) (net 8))
 (segment (start 115.794462 89) (end 122.494462 82.3) (width 0.254) (layer F.Cu) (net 8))
 (via (at 124.2 82.4) (size 0.6) (drill 0.4) (layers F.Cu B.Cu) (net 8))
 (segment (start 124.2 86.35) (end 124.2 82.4) (width 0.254) (layer B.Cu) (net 8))
 (segment (start 124.172999 82.372999) (end 124.2 82.4) (width 0.254) (layer F.Cu) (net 8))
 (segment (start 124.1 82.3) (end 124.2 82.4) (width 0.254) (layer F.Cu) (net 8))
 (segment (start 122.494462 82.3) (end 124.1 82.3) (width 0.254) (layer F.Cu) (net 8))
 (segment (start 125.45 86.35) (end 125.45 81.75) (width 0.254) (layer B.Cu) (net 7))
 (via (at 125.45 81.75) (size 0.6) (drill 0.4) (layers F.Cu B.Cu) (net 7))
 (segment (start 125.326198 81.626198) (end 125.45 81.75) (width 0.254) (layer F.Cu) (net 7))
 (segment (start 122.526198 81.626198) (end 125.326198 81.626198) (width 0.254) (layer F.Cu) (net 7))
 (segment (start 115.952396 88.2) (end 122.526198 81.626198) (width 0.254) (layer F.Cu) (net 7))
 (segment (start 112.5 88.2) (end 115.952396 88.2) (width 0.254) (layer F.Cu) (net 7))
 (via (at 126.6 81) (size 0.6) (drill 0.4) (layers F.Cu B.Cu) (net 6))
 (segment (start 126.7 81.1) (end 126.6 81) (width 0.254) (layer B.Cu) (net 6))
 (segment (start 126.7 86.35) (end 126.7 81.1) (width 0.254) (layer B.Cu) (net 6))
 (segment (start 126.594835 81.005165) (end 126.6 81) (width 0.254) (layer F.Cu) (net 6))
 (segment (start 122.505165 81.005165) (end 126.594835 81.005165) (width 0.254) (layer F.Cu) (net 6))
 (segment (start 116.11033 87.4) (end 122.505165 81.005165) (width 0.254) (layer F.Cu) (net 6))
 (segment (start 112.5 87.4) (end 116.11033 87.4) (width 0.254) (layer F.Cu) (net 6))
 (segment (start 127.95 80.35) (end 128 80.3) (width 0.254) (layer B.Cu) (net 5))
 (via (at 128 80.3) (size 0.6) (drill 0.4) (layers F.Cu B.Cu) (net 5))
 (segment (start 127.95 86.35) (end 127.95 80.35) (width 0.254) (layer B.Cu) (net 5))
 (segment (start 127.965868 80.334132) (end 128 80.3) (width 0.254) (layer F.Cu) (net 5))
 (segment (start 122.534132 80.334132) (end 127.965868 80.334132) (width 0.254) (layer F.Cu) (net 5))
 (segment (start 116.268264 86.6) (end 122.534132 80.334132) (width 0.254) (layer F.Cu) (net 5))
 (segment (start 112.5 86.6) (end 116.268264 86.6) (width 0.254) (layer F.Cu) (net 5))
 (via (at 129.1 79.7) (size 0.6) (drill 0.4) (layers F.Cu B.Cu) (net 4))
 (segment (start 129.2 79.8) (end 129.1 79.7) (width 0.254) (layer B.Cu) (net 4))
 (segment (start 129.2 86.35) (end 129.2 79.8) (width 0.254) (layer B.Cu) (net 4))
 (segment (start 129.072999 79.672999) (end 129.1 79.7) (width 0.254) (layer F.Cu) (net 4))
 (segment (start 127.699039 79.672999) (end 129.072999 79.672999) (width 0.254) (layer F.Cu) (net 4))
 (segment (start 127.658939 79.713099) (end 127.699039 79.672999) (width 0.254) (layer F.Cu) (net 4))
 (segment (start 122.513099 79.713099) (end 127.658939 79.713099) (width 0.254) (layer F.Cu) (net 4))
 (segment (start 116.426198 85.8) (end 122.513099 79.713099) (width 0.254) (layer F.Cu) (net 4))
 (segment (start 112.5 85.8) (end 116.426198 85.8) (width 0.254) (layer F.Cu) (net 4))
 (segment (start 112.5 85) (end 116.584132 85) (width 0.254) (layer F.Cu) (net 3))
 (segment (start 116.584132 85) (end 122.484132 79.1) (width 0.254) (layer F.Cu) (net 3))
 (via (at 130.5 79.1) (size 0.6) (drill 0.4) (layers F.Cu B.Cu) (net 3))
 (segment (start 130.45 79.15) (end 130.5 79.1) (width 0.254) (layer B.Cu) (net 3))
 (segment (start 130.45 86.35) (end 130.45 79.15) (width 0.254) (layer B.Cu) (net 3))
 (segment (start 130.472999 79.072999) (end 130.5 79.1) (width 0.254) (layer F.Cu) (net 3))
 (segment (start 128.772038 79.1) (end 128.799039 79.072999) (width 0.254) (layer F.Cu) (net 3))
 (segment (start 128.799039 79.072999) (end 130.472999 79.072999) (width 0.254) (layer F.Cu) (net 3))
 (segment (start 122.484132 79.1) (end 128.772038 79.1) (width 0.254) (layer F.Cu) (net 3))
 (segment (start 112.5 89) (end 116.584132 89) (width 0.254) (layer B.Cu) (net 18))
 (segment (start 116.584132 89) (end 122.484132 94.9) (width 0.254) (layer B.Cu) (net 18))
 (via (at 124.2 94.9) (size 0.6) (drill 0.4) (layers F.Cu B.Cu) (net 18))
 (segment (start 124.2 87.6) (end 124.2 94.9) (width 0.254) (layer F.Cu) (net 18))
 (segment (start 122.484132 94.9) (end 124.2 94.9) (width 0.254) (layer B.Cu) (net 18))
 (via (at 156 94.9) (size 0.6) (drill 0.4) (layers F.Cu B.Cu) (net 18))
 (segment (start 156 87.5) (end 156 94.9) (width 0.254) (layer F.Cu) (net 18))
 (via (at 142.5 94.9) (size 0.6) (drill 0.4) (layers F.Cu B.Cu) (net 18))
 (segment (start 142.5 87.5) (end 142.5 94.9) (width 0.254) (layer F.Cu) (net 18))
 (segment (start 142.472999 94.927001) (end 142.5 94.9) (width 0.254) (layer B.Cu) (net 18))
 (segment (start 124.427001 94.927001) (end 142.472999 94.927001) (width 0.254) (layer B.Cu) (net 18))
 (segment (start 124.4 94.9) (end 124.427001 94.927001) (width 0.254) (layer B.Cu) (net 18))
 (segment (start 124.2 94.9) (end 124.4 94.9) (width 0.254) (layer B.Cu) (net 18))
 (segment (start 155.972999 94.927001) (end 156 94.9) (width 0.254) (layer B.Cu) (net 18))
 (segment (start 142.527001 94.927001) (end 155.972999 94.927001) (width 0.254) (layer B.Cu) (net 18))
 (segment (start 142.5 94.9) (end 142.527001 94.927001) (width 0.254) (layer B.Cu) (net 18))
 (segment (start 112.5 83.4) (end 115.478594 83.4) (width 0.254) (layer B.Cu) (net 11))
 (segment (start 115.478594 83.4) (end 122.478594 90.4) (width 0.254) (layer B.Cu) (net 11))
 (segment (start 132.95 87.6) (end 132.95 90.25) (width 0.254) (layer F.Cu) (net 11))
 (via (at 132.95 90.25) (size 0.6) (drill 0.4) (layers F.Cu B.Cu) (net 11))
 (segment (start 132.8 90.4) (end 132.95 90.25) (width 0.254) (layer B.Cu) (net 11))
 (segment (start 122.478594 90.4) (end 132.8 90.4) (width 0.254) (layer B.Cu) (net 11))
 (segment (start 132.95 90.25) (end 133.55 90.25) (width 0.254) (layer F.Cu) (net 11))
 (segment (start 133.55 90.25) (end 135.7 88.1) (width 0.254) (layer F.Cu) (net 11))
 (segment (start 135.7 85.4) (end 136.6 84.5) (width 0.254) (layer F.Cu) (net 11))
 (segment (start 135.7 88.1) (end 135.7 85.4) (width 0.254) (layer F.Cu) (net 11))
 (segment (start 137 84.5) (end 137.04575 84.45425) (width 0.254) (layer F.Cu) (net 11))
 (segment (start 136.6 84.5) (end 137 84.5) (width 0.254) (layer F.Cu) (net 11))
 (segment (start 137.04575 84.45425) (end 142.85425 84.45425) (width 0.254) (layer F.Cu) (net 11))
 (segment (start 143.75 85.35) (end 143.75 86.25) (width 0.254) (layer F.Cu) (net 11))
 (segment (start 142.85425 84.45425) (end 143.75 85.35) (width 0.254) (layer F.Cu) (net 11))
 (segment (start 112.5 84.2) (end 115.636528 84.2) (width 0.254) (layer B.Cu) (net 12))
 (segment (start 115.636528 84.2) (end 122.436528 91) (width 0.254) (layer B.Cu) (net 12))
 (via (at 131.7 91.027) (size 0.6) (drill 0.4) (layers F.Cu B.Cu) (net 12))
 (segment (start 131.7 87.6) (end 131.7 91.027) (width 0.254) (layer F.Cu) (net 12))
 (segment (start 131.673 91) (end 131.7 91.027) (width 0.254) (layer B.Cu) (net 12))
 (segment (start 122.436528 91) (end 131.673 91) (width 0.254) (layer B.Cu) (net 12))
 (segment (start 131.7 91.027) (end 133.673 91.027) (width 0.254) (layer F.Cu) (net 12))
 (segment (start 133.673 91.027) (end 136.3 88.4) (width 0.254) (layer F.Cu) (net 12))
 (segment (start 137.2 85) (end 137.2 84.942067) (width 0.254) (layer F.Cu) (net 12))
 (segment (start 136.3 85.9) (end 137.2 85) (width 0.254) (layer F.Cu) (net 12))
 (segment (start 136.3 88.4) (end 136.3 85.9) (width 0.254) (layer F.Cu) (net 12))
 (segment (start 137.2 84.942067) (end 137.233807 84.90826) (width 0.254) (layer F.Cu) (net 12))
 (segment (start 137.233807 84.90826) (end 141.90826 84.90826) (width 0.254) (layer F.Cu) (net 12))
 (segment (start 142.5 85.5) (end 142.5 86.25) (width 0.254) (layer F.Cu) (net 12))
 (segment (start 141.90826 84.90826) (end 142.5 85.5) (width 0.254) (layer F.Cu) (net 12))
 (segment (start 112.5 84.2) (end 116.742066 84.2) (width 0.254) (layer F.Cu) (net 2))
 (segment (start 116.742066 84.2) (end 122.442066 78.5) (width 0.254) (layer F.Cu) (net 2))
 (via (at 131.7 78.5) (size 0.6) (drill 0.4) (layers F.Cu B.Cu) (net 2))
 (segment (start 131.7 86.35) (end 131.7 78.5) (width 0.254) (layer B.Cu) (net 2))
 (segment (start 131.672999 78.472999) (end 131.7 78.5) (width 0.254) (layer F.Cu) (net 2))
 (segment (start 130.199039 78.472999) (end 131.672999 78.472999) (width 0.254) (layer F.Cu) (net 2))
 (segment (start 130.172038 78.5) (end 130.199039 78.472999) (width 0.254) (layer F.Cu) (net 2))
 (segment (start 122.442066 78.5) (end 130.172038 78.5) (width 0.254) (layer F.Cu) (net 2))
 (segment (start 112.5 83.4) (end 116.9 83.4) (width 0.254) (layer F.Cu) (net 1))
 (segment (start 116.9 83.4) (end 122.5 77.8) (width 0.254) (layer F.Cu) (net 1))
 (via (at 132.9 77.8) (size 0.6) (drill 0.4) (layers F.Cu B.Cu) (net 1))
 (segment (start 132.95 77.85) (end 132.9 77.8) (width 0.254) (layer B.Cu) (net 1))
 (segment (start 132.95 86.35) (end 132.95 77.85) (width 0.254) (layer B.Cu) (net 1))
 (segment (start 124.9 77.8) (end 132.9 77.8) (width 0.254) (layer F.Cu) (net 1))
 (segment (start 122.5 77.8) (end 124.9 77.8) (width 0.254) (layer F.Cu) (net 1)))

